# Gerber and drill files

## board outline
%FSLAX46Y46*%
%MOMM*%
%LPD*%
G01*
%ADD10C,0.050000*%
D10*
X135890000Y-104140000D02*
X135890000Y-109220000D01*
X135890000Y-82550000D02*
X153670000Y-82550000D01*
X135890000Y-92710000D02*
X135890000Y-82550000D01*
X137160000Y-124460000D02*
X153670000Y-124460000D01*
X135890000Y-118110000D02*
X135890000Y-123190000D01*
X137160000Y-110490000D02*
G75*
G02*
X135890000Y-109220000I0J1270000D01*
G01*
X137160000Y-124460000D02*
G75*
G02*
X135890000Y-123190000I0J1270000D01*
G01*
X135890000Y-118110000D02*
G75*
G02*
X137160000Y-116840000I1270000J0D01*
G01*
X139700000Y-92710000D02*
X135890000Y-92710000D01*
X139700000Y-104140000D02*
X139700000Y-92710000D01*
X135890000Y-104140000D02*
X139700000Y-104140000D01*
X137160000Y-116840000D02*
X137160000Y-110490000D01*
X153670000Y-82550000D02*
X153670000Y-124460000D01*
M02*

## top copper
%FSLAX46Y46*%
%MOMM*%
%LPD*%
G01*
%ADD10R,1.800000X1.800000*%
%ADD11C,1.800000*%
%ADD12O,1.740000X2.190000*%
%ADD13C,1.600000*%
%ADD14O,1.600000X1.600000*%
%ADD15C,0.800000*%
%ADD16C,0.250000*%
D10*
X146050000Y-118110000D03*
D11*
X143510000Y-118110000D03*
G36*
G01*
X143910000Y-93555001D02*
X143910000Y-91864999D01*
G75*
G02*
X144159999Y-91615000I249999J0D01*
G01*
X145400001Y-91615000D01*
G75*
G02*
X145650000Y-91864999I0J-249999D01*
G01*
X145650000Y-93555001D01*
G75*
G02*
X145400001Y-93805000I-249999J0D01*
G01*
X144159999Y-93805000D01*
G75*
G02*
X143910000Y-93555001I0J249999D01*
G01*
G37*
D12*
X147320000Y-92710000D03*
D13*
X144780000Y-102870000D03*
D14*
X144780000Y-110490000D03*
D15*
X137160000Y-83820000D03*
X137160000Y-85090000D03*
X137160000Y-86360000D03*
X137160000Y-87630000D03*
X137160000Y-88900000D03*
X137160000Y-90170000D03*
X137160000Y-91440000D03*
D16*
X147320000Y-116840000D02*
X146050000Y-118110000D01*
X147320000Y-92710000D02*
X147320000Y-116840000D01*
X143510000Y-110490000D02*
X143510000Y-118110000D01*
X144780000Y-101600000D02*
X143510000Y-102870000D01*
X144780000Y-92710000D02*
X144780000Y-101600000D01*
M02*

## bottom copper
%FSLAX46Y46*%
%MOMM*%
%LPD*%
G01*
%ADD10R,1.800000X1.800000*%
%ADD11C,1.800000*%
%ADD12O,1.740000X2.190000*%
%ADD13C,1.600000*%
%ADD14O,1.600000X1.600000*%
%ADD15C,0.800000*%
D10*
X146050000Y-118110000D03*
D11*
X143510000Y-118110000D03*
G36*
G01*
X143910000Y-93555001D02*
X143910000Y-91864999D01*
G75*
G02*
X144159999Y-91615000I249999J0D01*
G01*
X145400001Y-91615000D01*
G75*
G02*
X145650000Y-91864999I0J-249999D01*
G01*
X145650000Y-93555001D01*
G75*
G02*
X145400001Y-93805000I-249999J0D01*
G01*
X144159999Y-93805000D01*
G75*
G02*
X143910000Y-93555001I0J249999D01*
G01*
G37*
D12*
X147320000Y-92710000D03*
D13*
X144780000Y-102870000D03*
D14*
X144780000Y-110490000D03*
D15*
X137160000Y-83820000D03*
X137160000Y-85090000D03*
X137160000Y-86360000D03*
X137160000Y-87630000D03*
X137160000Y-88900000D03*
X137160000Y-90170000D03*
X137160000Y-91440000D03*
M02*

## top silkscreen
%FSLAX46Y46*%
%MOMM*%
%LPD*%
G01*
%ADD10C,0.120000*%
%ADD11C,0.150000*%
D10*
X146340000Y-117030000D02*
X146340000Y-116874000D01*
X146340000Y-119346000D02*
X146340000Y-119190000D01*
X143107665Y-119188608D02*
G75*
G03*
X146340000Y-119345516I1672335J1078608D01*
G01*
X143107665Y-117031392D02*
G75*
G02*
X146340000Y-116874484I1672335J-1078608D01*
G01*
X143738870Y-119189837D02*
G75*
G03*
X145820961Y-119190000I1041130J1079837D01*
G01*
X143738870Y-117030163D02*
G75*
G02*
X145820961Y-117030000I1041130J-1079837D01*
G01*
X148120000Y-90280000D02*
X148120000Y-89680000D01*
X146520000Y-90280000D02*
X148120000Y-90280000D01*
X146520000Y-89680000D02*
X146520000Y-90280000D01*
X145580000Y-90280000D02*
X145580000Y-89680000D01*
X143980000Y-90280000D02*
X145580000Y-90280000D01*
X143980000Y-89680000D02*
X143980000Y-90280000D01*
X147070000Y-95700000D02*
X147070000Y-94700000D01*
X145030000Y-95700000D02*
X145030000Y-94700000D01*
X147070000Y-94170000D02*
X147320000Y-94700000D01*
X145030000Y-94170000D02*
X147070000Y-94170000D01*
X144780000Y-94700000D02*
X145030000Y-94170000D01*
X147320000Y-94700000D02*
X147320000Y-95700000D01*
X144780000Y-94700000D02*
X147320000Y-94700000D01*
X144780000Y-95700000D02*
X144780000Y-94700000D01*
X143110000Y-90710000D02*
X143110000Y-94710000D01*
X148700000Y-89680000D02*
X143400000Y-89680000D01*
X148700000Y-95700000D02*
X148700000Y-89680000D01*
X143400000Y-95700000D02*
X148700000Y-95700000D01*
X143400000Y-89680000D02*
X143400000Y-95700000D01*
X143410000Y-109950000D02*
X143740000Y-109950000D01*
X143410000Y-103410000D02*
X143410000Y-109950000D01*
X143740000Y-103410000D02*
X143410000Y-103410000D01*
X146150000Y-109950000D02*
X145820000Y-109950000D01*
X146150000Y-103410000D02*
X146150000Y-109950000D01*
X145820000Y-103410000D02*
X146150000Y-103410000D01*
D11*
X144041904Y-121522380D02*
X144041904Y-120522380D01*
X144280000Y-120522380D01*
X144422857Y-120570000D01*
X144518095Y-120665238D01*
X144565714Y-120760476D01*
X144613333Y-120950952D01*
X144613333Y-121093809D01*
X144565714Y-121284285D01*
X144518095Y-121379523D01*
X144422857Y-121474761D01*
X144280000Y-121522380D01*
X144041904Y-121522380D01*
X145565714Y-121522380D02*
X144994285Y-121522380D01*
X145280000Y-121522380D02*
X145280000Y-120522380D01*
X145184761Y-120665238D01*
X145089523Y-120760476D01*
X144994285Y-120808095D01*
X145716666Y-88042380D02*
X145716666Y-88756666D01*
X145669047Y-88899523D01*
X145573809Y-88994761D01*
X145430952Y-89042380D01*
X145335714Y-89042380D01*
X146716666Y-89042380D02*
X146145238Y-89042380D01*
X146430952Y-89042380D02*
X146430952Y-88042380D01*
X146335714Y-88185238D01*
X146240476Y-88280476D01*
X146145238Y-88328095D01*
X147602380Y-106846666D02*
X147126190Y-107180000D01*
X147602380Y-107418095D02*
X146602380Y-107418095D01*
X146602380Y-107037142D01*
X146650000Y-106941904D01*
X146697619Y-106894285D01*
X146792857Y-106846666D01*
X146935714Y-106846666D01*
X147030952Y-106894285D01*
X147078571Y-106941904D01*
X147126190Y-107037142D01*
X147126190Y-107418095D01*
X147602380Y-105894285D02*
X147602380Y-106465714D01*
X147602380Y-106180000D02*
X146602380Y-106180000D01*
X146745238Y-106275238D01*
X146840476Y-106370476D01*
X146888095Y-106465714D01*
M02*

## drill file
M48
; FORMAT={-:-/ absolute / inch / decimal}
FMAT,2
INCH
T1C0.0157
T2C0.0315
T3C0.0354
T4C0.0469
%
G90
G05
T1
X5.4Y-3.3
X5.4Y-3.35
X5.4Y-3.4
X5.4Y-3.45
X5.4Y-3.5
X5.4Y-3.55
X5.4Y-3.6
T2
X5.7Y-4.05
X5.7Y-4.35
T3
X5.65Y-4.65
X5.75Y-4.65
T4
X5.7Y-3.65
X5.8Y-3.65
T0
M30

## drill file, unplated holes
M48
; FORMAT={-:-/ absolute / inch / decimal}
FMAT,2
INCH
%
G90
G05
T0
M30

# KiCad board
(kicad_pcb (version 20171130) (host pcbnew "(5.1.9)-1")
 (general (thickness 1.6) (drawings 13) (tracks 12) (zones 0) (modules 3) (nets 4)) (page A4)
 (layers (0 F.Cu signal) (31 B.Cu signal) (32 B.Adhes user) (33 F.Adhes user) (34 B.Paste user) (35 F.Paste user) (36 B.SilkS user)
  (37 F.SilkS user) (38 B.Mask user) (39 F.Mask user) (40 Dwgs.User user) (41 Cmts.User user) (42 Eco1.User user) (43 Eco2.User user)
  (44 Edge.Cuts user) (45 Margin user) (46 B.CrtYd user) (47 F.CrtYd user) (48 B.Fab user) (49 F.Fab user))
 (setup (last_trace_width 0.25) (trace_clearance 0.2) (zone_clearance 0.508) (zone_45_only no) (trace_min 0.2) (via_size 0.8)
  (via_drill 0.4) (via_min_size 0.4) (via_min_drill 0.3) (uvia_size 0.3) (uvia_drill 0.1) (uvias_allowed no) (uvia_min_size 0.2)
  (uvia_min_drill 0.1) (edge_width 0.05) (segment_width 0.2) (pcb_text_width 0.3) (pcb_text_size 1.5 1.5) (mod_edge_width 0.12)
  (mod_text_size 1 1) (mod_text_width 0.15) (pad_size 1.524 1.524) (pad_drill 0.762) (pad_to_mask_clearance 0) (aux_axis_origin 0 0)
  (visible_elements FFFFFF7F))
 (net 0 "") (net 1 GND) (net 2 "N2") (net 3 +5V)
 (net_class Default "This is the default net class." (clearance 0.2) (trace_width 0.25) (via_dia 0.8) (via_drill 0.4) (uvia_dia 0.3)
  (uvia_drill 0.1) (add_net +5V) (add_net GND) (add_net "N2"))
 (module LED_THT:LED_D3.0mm (layer F.Cu) (at 146.05 118.11 180)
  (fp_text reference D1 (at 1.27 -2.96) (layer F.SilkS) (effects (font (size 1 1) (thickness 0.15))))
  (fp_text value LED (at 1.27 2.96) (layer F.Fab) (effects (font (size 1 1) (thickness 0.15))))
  (fp_line (start -0.29 1.08) (end -0.29 1.236) (layer F.SilkS) (width 0.12))
  (fp_line (start -0.29 -1.236) (end -0.29 -1.08) (layer F.SilkS) (width 0.12))
  (fp_arc (start 1.27 0) (end -0.29 -1.235516) (angle 108.8) (layer F.SilkS) (width 0.12))
  (fp_arc (start 1.27 0) (end -0.29 1.235516) (angle -108.8) (layer F.SilkS) (width 0.12))
  (fp_arc (start 1.27 0) (end 0.229039 -1.08) (angle 87.9) (layer F.SilkS) (width 0.12))
  (fp_arc (start 1.27 0) (end 0.229039 1.08) (angle -87.9) (layer F.SilkS) (width 0.12))
  (pad 1 thru_hole rect (at 0 0 180) (size 1.8 1.8) (drill 0.9) (layers *.Cu *.Mask) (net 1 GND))
  (pad 2 thru_hole circle (at 2.54 0 180) (size 1.8 1.8) (drill 0.9) (layers *.Cu *.Mask) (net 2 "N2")))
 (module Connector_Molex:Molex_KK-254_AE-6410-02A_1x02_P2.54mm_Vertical (layer F.Cu) (at 144.78 92.71)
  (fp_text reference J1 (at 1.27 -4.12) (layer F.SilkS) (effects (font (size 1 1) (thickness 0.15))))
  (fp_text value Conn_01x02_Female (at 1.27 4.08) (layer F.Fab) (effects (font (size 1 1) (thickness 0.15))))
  (fp_line (start 3.34 -2.43) (end 3.34 -3.03) (layer F.SilkS) (width 0.12))
  (fp_line (start 1.74 -2.43) (end 3.34 -2.43) (layer F.SilkS) (width 0.12))
  (fp_line (start 1.74 -3.03) (end 1.74 -2.43) (layer F.SilkS) (width 0.12))
  (fp_line (start 0.8 -2.43) (end 0.8 -3.03) (layer F.SilkS) (width 0.12))
  (fp_line (start -0.8 -2.43) (end 0.8 -2.43) (layer F.SilkS) (width 0.12))
  (fp_line (start -0.8 -3.03) (end -0.8 -2.43) (layer F.SilkS) (width 0.12))
  (fp_line (start 2.29 2.99) (end 2.29 1.99) (layer F.SilkS) (width 0.12))
  (fp_line (start 0.25 2.99) (end 0.25 1.99) (layer F.SilkS) (width 0.12))
  (fp_line (start 2.29 1.46) (end 2.54 1.99) (layer F.SilkS) (width 0.12))
  (fp_line (start 0.25 1.46) (end 2.29 1.46) (layer F.SilkS) (width 0.12))
  (fp_line (start 0 1.99) (end 0.25 1.46) (layer F.SilkS) (width 0.12))
  (fp_line (start 2.54 1.99) (end 2.54 2.99) (layer F.SilkS) (width 0.12))
  (fp_line (start 0 1.99) (end 2.54 1.99) (layer F.SilkS) (width 0.12))
  (fp_line (start 0 2.99) (end 0 1.99) (layer F.SilkS) (width 0.12))
  (fp_line (start -1.67 -2) (end -1.67 2) (layer F.SilkS) (width 0.12))
  (fp_line (start 3.92 -3.03) (end -1.38 -3.03) (layer F.SilkS) (width 0.12))
  (fp_line (start 3.92 2.99) (end 3.92 -3.03) (layer F.SilkS) (width 0.12))
  (fp_line (start -1.38 2.99) (end 3.92 2.99) (layer F.SilkS) (width 0.12))
  (fp_line (start -1.38 -3.03) (end -1.38 2.99) (layer F.SilkS) (width 0.12))
  (pad 1 thru_hole roundrect (at 0 0) (size 1.74 2.19) (drill 1.19) (layers *.Cu *.Mask) (roundrect_rratio 0.1436775862068966) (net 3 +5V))
  (pad 2 thru_hole oval (at 2.54 0) (size 1.74 2.19) (drill 1.19) (layers *.Cu *.Mask) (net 1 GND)))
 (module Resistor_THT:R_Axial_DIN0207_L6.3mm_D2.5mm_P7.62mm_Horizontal (layer F.Cu) (at 144.78 102.87 270)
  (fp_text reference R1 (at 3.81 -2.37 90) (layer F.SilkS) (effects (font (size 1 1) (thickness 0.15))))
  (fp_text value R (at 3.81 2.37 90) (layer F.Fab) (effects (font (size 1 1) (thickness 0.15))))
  (fp_line (start 7.08 1.37) (end 7.08 1.04) (layer F.SilkS) (width 0.12))
  (fp_line (start 0.54 1.37) (end 7.08 1.37) (layer F.SilkS) (width 0.12))
  (fp_line (start 0.54 1.04) (end 0.54 1.37) (layer F.SilkS) (width 0.12))
  (fp_line (start 7.08 -1.37) (end 7.08 -1.04) (layer F.SilkS) (width 0.12))
  (fp_line (start 0.54 -1.37) (end 7.08 -1.37) (layer F.SilkS) (width 0.12))
  (fp_line (start 0.54 -1.04) (end 0.54 -1.37) (layer F.SilkS) (width 0.12))
  (pad 1 thru_hole circle (at 0 0 270) (size 1.6 1.6) (drill 0.8) (layers *.Cu *.Mask) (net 3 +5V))
  (pad 2 thru_hole oval (at 7.62 0 270) (size 1.6 1.6) (drill 0.8) (layers *.Cu *.Mask) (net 2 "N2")))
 (gr_line (start 135.89 104.14) (end 135.89 109.22) (layer Edge.Cuts) (width 0.05))
 (gr_line (start 135.89 82.55) (end 153.67 82.55) (layer Edge.Cuts) (width 0.05))
 (gr_line (start 135.89 92.71) (end 135.89 82.55) (layer Edge.Cuts) (width 0.05))
 (gr_line (start 137.16 124.46) (end 153.67 124.46) (layer Edge.Cuts) (width 0.05))
 (gr_line (start 135.89 118.11) (end 135.89 123.19) (layer Edge.Cuts) (width 0.05))
 (gr_arc (start 137.16 109.22) (end 135.89 109.22) (angle -90) (layer Edge.Cuts) (width 0.05))
 (gr_arc (start 137.16 123.19) (end 135.89 123.19) (angle -90) (layer Edge.Cuts) (width 0.05))
 (gr_arc (start 137.16 118.11) (end 137.16 116.84) (angle -90) (layer Edge.Cuts) (width 0.05))
 (gr_line (start 139.7 92.71) (end 135.89 92.71) (layer Edge.Cuts) (width 0.05))
 (gr_line (start 139.7 104.14) (end 139.7 92.71) (layer Edge.Cuts) (width 0.05))
 (gr_line (start 135.89 104.14) (end 139.7 104.14) (layer Edge.Cuts) (width 0.05))
 (gr_line (start 137.16 116.84) (end 137.16 110.49) (layer Edge.Cuts) (width 0.05))
 (gr_line (start 153.67 82.55) (end 153.67 124.46) (layer Edge.Cuts) (width 0.05))
 (via (at 137.16 83.82) (size 0.8) (drill 0.4) (layers F.Cu B.Cu) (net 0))
 (via (at 137.16 85.09) (size 0.8) (drill 0.4) (layers F.Cu B.Cu) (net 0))
 (via (at 137.16 86.36) (size 0.8) (drill 0.4) (layers F.Cu B.Cu) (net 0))
 (via (at 137.16 87.63) (size 0.8) (drill 0.4) (layers F.Cu B.Cu) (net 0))
 (via (at 137.16 88.9) (size 0.8) (drill 0.4) (layers F.Cu B.Cu) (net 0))
 (via (at 137.16 90.17) (size 0.8) (drill 0.4) (layers F.Cu B.Cu) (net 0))
 (via (at 137.16 91.44) (size 0.8) (drill 0.4) (layers F.Cu B.Cu) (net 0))
 (segment (start 147.32 116.84) (end 146.05 118.11) (width 0.25) (layer F.Cu) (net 1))
 (segment (start 147.32 92.71) (end 147.32 116.84) (width 0.25) (layer F.Cu) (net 1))
 (segment (start 143.51 110.49) (end 143.51 118.11) (width 0.25) (layer F.Cu) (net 2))
 (segment (start 144.78 101.6) (end 143.51 102.87) (width 0.25) (layer F.Cu) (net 3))
 (segment (start 144.78 92.71) (end 144.78 101.6) (width 0.25) (layer F.Cu) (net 3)))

